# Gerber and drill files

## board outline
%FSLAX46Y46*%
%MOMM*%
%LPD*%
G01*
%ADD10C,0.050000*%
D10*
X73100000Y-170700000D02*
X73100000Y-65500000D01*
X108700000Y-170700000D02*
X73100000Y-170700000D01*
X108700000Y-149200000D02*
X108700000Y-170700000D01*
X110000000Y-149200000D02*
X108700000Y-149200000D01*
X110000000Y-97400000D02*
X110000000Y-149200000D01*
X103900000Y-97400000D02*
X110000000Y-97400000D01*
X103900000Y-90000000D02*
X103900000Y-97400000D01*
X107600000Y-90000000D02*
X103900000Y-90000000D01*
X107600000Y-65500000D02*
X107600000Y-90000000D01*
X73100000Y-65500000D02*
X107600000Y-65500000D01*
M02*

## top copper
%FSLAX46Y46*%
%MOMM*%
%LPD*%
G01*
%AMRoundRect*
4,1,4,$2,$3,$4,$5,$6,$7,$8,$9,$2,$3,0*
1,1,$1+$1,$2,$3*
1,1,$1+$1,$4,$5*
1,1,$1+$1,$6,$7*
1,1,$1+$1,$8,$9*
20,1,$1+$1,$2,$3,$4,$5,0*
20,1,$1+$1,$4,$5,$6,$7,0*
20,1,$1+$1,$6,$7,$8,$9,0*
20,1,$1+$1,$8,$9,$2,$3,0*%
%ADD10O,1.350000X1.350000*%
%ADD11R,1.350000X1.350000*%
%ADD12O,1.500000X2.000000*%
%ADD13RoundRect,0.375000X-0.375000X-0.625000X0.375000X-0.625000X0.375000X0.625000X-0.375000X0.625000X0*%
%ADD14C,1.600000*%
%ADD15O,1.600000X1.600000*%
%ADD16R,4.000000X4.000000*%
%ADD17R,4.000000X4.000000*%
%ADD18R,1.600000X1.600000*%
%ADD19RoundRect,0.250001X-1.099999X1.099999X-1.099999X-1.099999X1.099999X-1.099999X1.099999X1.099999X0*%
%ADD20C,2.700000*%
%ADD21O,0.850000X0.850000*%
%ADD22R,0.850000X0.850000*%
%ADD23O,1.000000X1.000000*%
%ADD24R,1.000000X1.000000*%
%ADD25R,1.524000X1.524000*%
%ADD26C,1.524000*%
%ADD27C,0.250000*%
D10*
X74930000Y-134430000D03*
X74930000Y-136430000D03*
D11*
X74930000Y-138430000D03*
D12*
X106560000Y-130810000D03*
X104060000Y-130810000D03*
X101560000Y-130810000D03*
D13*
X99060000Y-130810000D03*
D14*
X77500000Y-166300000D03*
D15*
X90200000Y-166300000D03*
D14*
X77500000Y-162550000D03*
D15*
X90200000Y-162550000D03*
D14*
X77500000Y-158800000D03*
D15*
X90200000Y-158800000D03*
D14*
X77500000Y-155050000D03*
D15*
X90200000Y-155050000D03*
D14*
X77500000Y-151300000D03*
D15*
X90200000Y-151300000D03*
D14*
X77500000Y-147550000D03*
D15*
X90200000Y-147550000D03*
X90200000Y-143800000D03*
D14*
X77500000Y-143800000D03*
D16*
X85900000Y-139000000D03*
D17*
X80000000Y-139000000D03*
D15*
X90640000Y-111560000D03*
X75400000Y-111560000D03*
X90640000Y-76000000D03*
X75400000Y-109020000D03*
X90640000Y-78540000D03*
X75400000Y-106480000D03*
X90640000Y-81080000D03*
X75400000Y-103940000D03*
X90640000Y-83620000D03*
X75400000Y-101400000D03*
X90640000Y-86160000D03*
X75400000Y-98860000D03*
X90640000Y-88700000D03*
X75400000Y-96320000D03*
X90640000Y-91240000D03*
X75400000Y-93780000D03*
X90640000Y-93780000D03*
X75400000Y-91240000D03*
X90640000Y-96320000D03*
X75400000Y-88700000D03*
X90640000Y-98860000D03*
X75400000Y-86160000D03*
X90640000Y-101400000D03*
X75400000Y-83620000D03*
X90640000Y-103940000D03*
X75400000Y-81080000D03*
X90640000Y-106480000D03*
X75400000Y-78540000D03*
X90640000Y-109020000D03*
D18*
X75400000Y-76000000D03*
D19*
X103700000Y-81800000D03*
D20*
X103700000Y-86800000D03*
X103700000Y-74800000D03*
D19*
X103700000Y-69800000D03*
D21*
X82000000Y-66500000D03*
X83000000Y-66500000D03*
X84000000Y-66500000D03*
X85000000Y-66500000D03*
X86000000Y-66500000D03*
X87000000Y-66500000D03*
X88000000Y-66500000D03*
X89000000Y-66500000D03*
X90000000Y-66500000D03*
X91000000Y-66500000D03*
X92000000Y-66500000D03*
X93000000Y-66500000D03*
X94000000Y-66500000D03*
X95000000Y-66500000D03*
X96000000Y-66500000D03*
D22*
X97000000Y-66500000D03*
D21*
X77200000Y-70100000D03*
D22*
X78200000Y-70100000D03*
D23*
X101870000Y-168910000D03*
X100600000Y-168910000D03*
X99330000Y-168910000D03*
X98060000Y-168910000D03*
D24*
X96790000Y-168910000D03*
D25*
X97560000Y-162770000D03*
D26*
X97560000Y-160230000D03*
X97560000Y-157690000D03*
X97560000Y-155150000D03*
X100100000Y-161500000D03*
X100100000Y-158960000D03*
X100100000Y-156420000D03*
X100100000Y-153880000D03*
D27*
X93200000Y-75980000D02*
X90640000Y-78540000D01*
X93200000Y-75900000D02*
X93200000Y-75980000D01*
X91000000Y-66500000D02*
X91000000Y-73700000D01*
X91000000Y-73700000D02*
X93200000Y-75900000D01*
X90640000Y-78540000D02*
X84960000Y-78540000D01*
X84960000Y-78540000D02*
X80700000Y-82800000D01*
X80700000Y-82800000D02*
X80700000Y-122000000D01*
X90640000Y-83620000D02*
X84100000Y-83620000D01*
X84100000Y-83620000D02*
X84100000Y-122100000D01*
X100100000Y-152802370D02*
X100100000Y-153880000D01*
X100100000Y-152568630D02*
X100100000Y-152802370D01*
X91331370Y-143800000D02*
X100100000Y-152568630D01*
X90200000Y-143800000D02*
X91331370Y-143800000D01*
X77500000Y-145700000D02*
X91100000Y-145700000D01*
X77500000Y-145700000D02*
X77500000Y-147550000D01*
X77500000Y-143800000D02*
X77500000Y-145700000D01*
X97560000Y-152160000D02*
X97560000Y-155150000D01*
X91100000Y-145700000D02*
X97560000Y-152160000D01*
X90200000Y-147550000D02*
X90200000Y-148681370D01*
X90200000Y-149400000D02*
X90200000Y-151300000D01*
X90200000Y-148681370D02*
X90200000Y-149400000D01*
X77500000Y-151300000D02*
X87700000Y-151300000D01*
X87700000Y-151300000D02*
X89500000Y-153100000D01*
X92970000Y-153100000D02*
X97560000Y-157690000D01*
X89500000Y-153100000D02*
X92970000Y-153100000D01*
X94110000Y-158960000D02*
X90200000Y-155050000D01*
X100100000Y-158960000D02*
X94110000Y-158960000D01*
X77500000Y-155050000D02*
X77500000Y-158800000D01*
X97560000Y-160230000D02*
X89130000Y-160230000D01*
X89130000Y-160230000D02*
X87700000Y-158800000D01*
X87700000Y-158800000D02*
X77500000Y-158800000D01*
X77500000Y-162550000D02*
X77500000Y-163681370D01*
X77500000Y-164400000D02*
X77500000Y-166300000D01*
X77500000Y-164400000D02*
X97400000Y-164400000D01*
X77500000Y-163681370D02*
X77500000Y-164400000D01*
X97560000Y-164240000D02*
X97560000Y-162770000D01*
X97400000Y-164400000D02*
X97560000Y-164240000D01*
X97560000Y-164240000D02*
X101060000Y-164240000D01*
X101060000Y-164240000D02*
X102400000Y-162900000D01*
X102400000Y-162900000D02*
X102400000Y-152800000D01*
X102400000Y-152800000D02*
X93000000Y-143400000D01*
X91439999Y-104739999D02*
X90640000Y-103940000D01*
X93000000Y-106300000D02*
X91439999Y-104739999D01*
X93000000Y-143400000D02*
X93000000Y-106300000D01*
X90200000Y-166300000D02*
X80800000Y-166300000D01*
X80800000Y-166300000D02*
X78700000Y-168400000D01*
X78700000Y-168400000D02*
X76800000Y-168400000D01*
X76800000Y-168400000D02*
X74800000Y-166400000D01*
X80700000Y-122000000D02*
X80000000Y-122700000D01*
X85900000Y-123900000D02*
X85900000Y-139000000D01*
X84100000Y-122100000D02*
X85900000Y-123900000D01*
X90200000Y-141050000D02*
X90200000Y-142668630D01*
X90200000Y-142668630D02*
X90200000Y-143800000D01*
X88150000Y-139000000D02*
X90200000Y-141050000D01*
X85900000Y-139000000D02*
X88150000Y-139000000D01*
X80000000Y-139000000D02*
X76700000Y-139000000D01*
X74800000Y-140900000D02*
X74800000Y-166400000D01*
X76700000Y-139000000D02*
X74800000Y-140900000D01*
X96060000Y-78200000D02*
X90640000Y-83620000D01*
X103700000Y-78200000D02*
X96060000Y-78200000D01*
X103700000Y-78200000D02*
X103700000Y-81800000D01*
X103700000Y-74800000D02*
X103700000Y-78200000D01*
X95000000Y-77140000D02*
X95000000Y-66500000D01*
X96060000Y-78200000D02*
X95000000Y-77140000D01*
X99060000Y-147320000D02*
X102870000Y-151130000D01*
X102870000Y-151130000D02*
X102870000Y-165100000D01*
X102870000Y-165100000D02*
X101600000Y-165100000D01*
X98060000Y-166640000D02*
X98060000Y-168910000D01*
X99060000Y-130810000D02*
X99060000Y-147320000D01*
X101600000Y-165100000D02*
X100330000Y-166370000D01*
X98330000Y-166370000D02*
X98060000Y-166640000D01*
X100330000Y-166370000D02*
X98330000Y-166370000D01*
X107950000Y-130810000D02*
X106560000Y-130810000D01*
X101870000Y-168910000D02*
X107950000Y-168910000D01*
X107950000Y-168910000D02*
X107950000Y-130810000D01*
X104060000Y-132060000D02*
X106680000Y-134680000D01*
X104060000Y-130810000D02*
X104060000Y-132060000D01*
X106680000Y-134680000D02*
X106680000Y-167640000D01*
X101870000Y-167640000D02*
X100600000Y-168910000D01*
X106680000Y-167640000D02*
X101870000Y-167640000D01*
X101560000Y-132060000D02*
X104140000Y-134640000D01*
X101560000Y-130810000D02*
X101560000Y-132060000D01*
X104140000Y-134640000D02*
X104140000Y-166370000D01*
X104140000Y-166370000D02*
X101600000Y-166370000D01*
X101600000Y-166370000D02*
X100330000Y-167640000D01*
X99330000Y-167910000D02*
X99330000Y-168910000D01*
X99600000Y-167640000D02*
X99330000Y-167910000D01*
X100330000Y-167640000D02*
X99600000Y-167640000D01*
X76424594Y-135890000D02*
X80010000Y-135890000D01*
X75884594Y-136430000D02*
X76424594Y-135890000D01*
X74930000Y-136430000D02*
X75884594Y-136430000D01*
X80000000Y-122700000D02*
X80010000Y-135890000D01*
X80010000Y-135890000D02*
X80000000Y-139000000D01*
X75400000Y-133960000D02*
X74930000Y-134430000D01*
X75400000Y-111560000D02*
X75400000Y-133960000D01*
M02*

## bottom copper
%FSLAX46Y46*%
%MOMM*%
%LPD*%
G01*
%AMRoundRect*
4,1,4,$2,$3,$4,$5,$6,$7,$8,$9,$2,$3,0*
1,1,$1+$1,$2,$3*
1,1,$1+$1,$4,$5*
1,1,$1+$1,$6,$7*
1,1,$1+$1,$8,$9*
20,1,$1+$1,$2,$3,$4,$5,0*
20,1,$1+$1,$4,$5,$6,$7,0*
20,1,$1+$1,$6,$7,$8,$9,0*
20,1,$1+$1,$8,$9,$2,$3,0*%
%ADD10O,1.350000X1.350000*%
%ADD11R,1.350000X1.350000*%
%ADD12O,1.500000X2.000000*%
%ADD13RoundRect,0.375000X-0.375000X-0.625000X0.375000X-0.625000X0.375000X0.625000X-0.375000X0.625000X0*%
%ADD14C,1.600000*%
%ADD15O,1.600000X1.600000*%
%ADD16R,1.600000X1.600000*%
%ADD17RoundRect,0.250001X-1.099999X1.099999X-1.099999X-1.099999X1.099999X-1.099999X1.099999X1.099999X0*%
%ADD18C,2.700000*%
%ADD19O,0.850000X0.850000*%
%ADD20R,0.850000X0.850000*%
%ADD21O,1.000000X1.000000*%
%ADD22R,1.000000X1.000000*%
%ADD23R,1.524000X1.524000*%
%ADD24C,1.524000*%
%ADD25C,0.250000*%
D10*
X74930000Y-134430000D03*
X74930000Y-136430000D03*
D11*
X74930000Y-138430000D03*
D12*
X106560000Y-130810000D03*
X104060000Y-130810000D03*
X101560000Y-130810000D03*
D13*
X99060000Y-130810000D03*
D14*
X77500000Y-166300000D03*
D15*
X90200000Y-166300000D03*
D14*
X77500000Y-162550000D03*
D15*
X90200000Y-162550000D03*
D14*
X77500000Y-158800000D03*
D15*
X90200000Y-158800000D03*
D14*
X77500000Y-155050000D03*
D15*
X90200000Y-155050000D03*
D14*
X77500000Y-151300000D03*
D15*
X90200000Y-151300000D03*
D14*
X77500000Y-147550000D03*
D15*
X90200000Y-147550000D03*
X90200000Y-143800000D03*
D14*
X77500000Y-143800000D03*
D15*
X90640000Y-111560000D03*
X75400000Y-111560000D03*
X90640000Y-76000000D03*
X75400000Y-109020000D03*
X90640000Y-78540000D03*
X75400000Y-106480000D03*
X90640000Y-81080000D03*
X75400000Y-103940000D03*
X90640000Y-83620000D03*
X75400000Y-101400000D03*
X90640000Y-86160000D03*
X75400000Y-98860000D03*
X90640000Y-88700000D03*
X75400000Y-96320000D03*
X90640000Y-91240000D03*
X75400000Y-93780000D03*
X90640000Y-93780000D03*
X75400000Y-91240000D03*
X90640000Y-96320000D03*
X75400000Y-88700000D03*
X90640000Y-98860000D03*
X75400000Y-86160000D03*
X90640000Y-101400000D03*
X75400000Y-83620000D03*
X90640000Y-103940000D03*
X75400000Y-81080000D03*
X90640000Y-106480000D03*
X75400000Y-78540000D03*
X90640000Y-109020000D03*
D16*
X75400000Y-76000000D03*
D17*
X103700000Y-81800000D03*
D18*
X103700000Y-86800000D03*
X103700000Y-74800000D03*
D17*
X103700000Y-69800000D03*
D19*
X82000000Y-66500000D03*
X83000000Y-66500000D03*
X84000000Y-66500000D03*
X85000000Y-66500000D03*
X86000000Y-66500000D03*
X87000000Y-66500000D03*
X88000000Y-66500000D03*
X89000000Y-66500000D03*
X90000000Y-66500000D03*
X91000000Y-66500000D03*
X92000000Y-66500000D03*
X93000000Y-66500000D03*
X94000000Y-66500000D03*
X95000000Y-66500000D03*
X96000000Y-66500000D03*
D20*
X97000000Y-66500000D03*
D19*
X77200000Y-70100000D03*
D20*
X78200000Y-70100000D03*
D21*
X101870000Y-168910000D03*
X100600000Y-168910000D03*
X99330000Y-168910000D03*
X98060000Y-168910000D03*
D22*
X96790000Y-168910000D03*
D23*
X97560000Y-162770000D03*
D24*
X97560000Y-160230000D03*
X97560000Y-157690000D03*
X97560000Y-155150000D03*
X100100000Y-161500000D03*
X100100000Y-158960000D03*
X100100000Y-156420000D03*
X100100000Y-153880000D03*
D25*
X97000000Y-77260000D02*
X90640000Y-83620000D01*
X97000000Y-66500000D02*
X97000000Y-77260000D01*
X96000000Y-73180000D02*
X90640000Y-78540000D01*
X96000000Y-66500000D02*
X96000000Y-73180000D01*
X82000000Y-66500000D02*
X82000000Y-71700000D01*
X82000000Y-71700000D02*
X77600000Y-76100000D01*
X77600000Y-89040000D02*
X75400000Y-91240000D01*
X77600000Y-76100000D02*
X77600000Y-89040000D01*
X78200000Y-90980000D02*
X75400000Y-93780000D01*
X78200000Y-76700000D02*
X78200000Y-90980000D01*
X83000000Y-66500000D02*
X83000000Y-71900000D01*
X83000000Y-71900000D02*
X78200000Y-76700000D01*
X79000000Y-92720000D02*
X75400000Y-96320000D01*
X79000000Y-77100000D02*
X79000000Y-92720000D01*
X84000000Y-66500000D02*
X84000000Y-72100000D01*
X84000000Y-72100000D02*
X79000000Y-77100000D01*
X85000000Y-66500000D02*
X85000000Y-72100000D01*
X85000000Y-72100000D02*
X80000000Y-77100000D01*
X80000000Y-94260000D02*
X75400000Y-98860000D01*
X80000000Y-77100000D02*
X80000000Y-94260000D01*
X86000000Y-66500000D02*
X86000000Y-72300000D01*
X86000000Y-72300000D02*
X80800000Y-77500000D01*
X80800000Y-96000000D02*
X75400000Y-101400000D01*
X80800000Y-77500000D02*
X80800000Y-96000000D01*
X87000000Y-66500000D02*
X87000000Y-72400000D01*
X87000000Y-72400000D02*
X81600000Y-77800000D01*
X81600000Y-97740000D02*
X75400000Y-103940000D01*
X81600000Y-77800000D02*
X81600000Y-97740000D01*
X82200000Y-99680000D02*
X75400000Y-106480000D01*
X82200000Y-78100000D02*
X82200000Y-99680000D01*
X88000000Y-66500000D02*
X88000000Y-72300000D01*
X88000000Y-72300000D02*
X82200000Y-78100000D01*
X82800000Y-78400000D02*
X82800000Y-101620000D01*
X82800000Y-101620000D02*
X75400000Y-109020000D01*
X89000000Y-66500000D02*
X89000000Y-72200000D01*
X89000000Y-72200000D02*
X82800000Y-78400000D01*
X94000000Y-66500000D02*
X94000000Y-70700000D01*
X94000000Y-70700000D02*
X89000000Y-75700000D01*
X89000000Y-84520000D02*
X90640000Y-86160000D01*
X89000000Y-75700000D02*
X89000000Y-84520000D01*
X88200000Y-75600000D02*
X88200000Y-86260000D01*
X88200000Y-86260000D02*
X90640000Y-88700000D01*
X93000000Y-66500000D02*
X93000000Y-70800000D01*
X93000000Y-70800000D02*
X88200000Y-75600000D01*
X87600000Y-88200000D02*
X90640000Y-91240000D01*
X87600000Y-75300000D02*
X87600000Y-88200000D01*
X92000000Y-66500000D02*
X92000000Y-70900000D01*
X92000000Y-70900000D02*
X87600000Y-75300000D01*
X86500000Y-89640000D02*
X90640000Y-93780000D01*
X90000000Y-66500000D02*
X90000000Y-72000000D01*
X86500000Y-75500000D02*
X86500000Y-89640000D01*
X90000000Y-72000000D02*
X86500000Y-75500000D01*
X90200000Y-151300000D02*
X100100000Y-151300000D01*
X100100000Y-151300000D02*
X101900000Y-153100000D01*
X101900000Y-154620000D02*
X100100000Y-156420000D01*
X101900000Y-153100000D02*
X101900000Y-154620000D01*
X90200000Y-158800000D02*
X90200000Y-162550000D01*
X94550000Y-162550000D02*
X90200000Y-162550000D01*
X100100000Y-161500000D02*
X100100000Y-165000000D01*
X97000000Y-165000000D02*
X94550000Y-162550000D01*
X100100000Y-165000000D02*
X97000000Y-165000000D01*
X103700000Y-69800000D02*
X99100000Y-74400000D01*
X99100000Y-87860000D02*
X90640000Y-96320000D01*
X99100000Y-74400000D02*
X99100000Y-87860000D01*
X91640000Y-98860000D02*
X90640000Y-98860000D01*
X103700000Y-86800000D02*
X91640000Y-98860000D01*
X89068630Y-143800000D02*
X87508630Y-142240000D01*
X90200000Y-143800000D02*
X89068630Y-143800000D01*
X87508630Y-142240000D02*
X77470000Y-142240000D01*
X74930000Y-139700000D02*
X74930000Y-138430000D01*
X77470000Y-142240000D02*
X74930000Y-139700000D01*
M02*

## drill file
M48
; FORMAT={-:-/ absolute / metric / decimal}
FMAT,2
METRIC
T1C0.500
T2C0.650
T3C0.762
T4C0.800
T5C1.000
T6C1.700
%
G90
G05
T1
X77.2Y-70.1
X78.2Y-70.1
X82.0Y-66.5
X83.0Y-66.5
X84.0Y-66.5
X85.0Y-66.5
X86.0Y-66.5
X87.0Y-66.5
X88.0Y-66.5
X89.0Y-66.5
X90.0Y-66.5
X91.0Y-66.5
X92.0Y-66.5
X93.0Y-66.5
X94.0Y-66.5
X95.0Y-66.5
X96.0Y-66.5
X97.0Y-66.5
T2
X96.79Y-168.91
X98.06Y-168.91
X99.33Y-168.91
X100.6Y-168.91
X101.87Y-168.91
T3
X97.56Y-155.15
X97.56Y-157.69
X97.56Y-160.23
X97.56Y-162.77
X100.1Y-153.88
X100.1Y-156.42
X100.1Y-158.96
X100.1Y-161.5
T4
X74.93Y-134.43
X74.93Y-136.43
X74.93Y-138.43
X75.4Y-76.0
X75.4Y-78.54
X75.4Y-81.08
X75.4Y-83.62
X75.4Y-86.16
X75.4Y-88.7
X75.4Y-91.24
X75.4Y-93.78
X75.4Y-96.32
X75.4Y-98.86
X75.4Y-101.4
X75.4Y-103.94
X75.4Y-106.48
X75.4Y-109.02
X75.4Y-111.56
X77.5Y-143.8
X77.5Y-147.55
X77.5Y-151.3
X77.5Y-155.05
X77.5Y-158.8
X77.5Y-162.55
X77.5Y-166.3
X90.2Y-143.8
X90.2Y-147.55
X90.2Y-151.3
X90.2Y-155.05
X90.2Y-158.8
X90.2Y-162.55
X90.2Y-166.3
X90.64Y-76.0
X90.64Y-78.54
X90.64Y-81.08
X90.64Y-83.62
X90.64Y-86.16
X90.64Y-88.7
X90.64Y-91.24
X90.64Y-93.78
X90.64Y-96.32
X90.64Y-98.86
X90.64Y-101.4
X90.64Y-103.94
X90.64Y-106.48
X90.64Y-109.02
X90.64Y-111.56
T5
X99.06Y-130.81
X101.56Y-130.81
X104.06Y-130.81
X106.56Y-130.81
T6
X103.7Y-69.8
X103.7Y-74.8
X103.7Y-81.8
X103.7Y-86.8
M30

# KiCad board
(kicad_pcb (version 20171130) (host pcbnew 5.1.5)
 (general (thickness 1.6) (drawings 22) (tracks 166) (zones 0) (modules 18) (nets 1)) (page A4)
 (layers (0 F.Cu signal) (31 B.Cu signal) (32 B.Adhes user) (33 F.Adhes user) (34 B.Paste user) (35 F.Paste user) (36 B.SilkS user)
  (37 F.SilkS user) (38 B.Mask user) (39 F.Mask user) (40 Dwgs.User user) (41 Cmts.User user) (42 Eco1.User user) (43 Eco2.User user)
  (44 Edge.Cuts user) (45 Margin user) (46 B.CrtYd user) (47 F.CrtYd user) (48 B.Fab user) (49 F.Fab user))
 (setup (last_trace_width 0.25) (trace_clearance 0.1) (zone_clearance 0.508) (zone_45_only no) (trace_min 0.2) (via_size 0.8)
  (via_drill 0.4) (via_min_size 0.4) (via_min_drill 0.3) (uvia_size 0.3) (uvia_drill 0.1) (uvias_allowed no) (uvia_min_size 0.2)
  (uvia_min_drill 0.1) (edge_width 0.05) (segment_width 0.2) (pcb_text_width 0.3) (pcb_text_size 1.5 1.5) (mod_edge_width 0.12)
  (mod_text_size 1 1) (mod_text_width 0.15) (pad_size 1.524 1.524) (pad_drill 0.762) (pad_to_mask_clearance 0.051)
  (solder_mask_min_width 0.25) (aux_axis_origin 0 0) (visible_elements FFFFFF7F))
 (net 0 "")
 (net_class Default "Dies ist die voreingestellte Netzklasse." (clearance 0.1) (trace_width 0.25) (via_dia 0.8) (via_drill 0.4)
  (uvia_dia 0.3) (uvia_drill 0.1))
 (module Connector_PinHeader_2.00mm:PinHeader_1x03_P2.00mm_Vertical (layer F.Cu) (at 74.93 138.43 180)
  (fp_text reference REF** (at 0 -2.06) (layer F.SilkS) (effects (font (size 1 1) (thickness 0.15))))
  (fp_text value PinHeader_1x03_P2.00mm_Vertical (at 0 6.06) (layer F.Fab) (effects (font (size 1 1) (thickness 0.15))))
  (pad 3 thru_hole oval (at 0 4 180) (size 1.35 1.35) (drill 0.8) (layers *.Cu *.Mask))
  (pad 2 thru_hole oval (at 0 2 180) (size 1.35 1.35) (drill 0.8) (layers *.Cu *.Mask))
  (pad 1 thru_hole rect (at 0 0 180) (size 1.35 1.35) (drill 0.8) (layers *.Cu *.Mask)))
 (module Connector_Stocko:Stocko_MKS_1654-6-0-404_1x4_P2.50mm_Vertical (layer F.Cu) (at 99.06 130.81)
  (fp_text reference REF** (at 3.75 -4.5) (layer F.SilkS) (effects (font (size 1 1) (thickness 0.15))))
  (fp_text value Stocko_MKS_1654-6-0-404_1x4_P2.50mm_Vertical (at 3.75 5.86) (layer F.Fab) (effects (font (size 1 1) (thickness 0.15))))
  (pad 4 thru_hole oval (at 7.5 0) (size 1.5 2) (drill 1) (layers *.Cu *.Mask))
  (pad 3 thru_hole oval (at 5 0) (size 1.5 2) (drill 1) (layers *.Cu *.Mask))
  (pad 2 thru_hole oval (at 2.5 0) (size 1.5 2) (drill 1) (layers *.Cu *.Mask))
  (pad 1 thru_hole roundrect (at 0 0) (size 1.5 2) (drill 1) (layers *.Cu *.Mask) (roundrect_rratio 0.25)))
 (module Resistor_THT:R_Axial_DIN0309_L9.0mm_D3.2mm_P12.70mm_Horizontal (layer F.Cu) (at 77.5 166.3)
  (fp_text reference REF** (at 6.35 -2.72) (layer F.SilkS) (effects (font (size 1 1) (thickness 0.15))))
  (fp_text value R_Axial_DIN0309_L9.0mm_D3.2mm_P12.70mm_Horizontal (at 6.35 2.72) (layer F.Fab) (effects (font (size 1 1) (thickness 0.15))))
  (pad 1 thru_hole circle (at 0 0) (size 1.6 1.6) (drill 0.8) (layers *.Cu *.Mask))
  (pad 2 thru_hole oval (at 12.7 0) (size 1.6 1.6) (drill 0.8) (layers *.Cu *.Mask)))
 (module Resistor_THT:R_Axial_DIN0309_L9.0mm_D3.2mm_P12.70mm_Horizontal (layer F.Cu) (at 77.5 162.55)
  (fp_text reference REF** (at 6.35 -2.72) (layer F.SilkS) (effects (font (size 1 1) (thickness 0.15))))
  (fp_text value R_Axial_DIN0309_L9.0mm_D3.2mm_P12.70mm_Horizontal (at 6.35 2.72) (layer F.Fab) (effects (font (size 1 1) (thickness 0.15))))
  (pad 1 thru_hole circle (at 0 0) (size 1.6 1.6) (drill 0.8) (layers *.Cu *.Mask))
  (pad 2 thru_hole oval (at 12.7 0) (size 1.6 1.6) (drill 0.8) (layers *.Cu *.Mask)))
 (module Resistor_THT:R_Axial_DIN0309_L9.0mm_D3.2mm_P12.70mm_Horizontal (layer F.Cu) (at 77.5 158.8)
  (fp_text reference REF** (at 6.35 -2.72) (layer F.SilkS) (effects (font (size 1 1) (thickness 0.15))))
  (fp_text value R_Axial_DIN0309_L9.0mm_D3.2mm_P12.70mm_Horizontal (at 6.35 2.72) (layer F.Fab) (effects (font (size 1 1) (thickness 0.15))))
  (pad 1 thru_hole circle (at 0 0) (size 1.6 1.6) (drill 0.8) (layers *.Cu *.Mask))
  (pad 2 thru_hole oval (at 12.7 0) (size 1.6 1.6) (drill 0.8) (layers *.Cu *.Mask)))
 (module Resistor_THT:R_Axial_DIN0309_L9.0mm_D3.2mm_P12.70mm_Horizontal (layer F.Cu) (at 77.5 155.05)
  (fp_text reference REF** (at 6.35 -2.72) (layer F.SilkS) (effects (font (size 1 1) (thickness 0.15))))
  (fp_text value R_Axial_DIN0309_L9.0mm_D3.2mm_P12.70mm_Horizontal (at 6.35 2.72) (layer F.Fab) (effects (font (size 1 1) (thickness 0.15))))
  (pad 1 thru_hole circle (at 0 0) (size 1.6 1.6) (drill 0.8) (layers *.Cu *.Mask))
  (pad 2 thru_hole oval (at 12.7 0) (size 1.6 1.6) (drill 0.8) (layers *.Cu *.Mask)))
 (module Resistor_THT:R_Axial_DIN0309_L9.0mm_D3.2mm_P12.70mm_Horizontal (layer F.Cu) (at 77.5 151.3)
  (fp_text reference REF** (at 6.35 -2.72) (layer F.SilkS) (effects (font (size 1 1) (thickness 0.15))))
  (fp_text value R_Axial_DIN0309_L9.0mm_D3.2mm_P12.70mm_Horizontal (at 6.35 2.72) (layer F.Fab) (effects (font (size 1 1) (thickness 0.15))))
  (pad 1 thru_hole circle (at 0 0) (size 1.6 1.6) (drill 0.8) (layers *.Cu *.Mask))
  (pad 2 thru_hole oval (at 12.7 0) (size 1.6 1.6) (drill 0.8) (layers *.Cu *.Mask)))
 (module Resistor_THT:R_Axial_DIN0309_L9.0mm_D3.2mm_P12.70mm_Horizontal (layer F.Cu) (at 77.5 147.55)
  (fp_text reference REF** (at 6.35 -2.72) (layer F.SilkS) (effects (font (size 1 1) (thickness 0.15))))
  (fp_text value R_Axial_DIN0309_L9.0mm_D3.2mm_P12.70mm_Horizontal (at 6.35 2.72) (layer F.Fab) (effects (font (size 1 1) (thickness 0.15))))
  (pad 1 thru_hole circle (at 0 0) (size 1.6 1.6) (drill 0.8) (layers *.Cu *.Mask))
  (pad 2 thru_hole oval (at 12.7 0) (size 1.6 1.6) (drill 0.8) (layers *.Cu *.Mask)))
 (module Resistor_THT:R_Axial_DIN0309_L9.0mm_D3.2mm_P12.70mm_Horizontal (layer F.Cu) (at 77.5 143.8)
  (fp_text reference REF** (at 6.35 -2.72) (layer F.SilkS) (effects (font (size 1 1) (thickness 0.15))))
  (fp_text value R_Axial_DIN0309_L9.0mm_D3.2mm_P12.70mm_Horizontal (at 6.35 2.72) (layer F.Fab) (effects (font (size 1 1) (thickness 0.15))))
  (pad 2 thru_hole oval (at 12.7 0) (size 1.6 1.6) (drill 0.8) (layers *.Cu *.Mask))
  (pad 1 thru_hole circle (at 0 0) (size 1.6 1.6) (drill 0.8) (layers *.Cu *.Mask)))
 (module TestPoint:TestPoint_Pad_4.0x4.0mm (layer F.Cu) (at 85.9 139)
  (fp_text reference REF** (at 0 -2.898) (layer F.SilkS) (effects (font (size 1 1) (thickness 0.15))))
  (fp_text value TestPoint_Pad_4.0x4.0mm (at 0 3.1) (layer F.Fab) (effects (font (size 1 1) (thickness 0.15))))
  (pad + connect rect (at 0 0) (size 4 4) (layers F.Cu F.Mask)))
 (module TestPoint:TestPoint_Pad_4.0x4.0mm (layer F.Cu) (at 80 139)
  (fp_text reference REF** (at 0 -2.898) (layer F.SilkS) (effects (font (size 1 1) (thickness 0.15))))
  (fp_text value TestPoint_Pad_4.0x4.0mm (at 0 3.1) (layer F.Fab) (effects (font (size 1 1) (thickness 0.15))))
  (pad - smd rect (at 0 0) (size 4 4) (layers F.Cu F.Mask)))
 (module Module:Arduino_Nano (layer F.Cu) (at 75.4 76)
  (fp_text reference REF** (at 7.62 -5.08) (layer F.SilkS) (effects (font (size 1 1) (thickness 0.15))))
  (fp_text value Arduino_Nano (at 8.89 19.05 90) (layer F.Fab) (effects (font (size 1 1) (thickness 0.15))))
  (pad 16 thru_hole oval (at 15.24 35.56) (size 1.6 1.6) (drill 0.8) (layers *.Cu *.Mask))
  (pad 15 thru_hole oval (at 0 35.56) (size 1.6 1.6) (drill 0.8) (layers *.Cu *.Mask))
  (pad 30 thru_hole oval (at 15.24 0) (size 1.6 1.6) (drill 0.8) (layers *.Cu *.Mask))
  (pad 14 thru_hole oval (at 0 33.02) (size 1.6 1.6) (drill 0.8) (layers *.Cu *.Mask))
  (pad 29 thru_hole oval (at 15.24 2.54) (size 1.6 1.6) (drill 0.8) (layers *.Cu *.Mask))
  (pad 13 thru_hole oval (at 0 30.48) (size 1.6 1.6) (drill 0.8) (layers *.Cu *.Mask))
  (pad 28 thru_hole oval (at 15.24 5.08) (size 1.6 1.6) (drill 0.8) (layers *.Cu *.Mask))
  (pad 12 thru_hole oval (at 0 27.94) (size 1.6 1.6) (drill 0.8) (layers *.Cu *.Mask))
  (pad 27 thru_hole oval (at 15.24 7.62) (size 1.6 1.6) (drill 0.8) (layers *.Cu *.Mask))
  (pad 11 thru_hole oval (at 0 25.4) (size 1.6 1.6) (drill 0.8) (layers *.Cu *.Mask))
  (pad 26 thru_hole oval (at 15.24 10.16) (size 1.6 1.6) (drill 0.8) (layers *.Cu *.Mask))
  (pad 10 thru_hole oval (at 0 22.86) (size 1.6 1.6) (drill 0.8) (layers *.Cu *.Mask))
  (pad 25 thru_hole oval (at 15.24 12.7) (size 1.6 1.6) (drill 0.8) (layers *.Cu *.Mask))
  (pad 9 thru_hole oval (at 0 20.32) (size 1.6 1.6) (drill 0.8) (layers *.Cu *.Mask))
  (pad 24 thru_hole oval (at 15.24 15.24) (size 1.6 1.6) (drill 0.8) (layers *.Cu *.Mask))
  (pad 8 thru_hole oval (at 0 17.78) (size 1.6 1.6) (drill 0.8) (layers *.Cu *.Mask))
  (pad 23 thru_hole oval (at 15.24 17.78) (size 1.6 1.6) (drill 0.8) (layers *.Cu *.Mask))
  (pad 7 thru_hole oval (at 0 15.24) (size 1.6 1.6) (drill 0.8) (layers *.Cu *.Mask))
  (pad 22 thru_hole oval (at 15.24 20.32) (size 1.6 1.6) (drill 0.8) (layers *.Cu *.Mask))
  (pad 6 thru_hole oval (at 0 12.7) (size 1.6 1.6) (drill 0.8) (layers *.Cu *.Mask))
  (pad 21 thru_hole oval (at 15.24 22.86) (size 1.6 1.6) (drill 0.8) (layers *.Cu *.Mask))
  (pad 5 thru_hole oval (at 0 10.16) (size 1.6 1.6) (drill 0.8) (layers *.Cu *.Mask))
  (pad 20 thru_hole oval (at 15.24 25.4) (size 1.6 1.6) (drill 0.8) (layers *.Cu *.Mask))
  (pad 4 thru_hole oval (at 0 7.62) (size 1.6 1.6) (drill 0.8) (layers *.Cu *.Mask))
  (pad 19 thru_hole oval (at 15.24 27.94) (size 1.6 1.6) (drill 0.8) (layers *.Cu *.Mask))
  (pad 3 thru_hole oval (at 0 5.08) (size 1.6 1.6) (drill 0.8) (layers *.Cu *.Mask))
  (pad 18 thru_hole oval (at 15.24 30.48) (size 1.6 1.6) (drill 0.8) (layers *.Cu *.Mask))
  (pad 2 thru_hole oval (at 0 2.54) (size 1.6 1.6) (drill 0.8) (layers *.Cu *.Mask))
  (pad 17 thru_hole oval (at 15.24 33.02) (size 1.6 1.6) (drill 0.8) (layers *.Cu *.Mask))
  (pad 1 thru_hole rect (at 0 0) (size 1.6 1.6) (drill 0.8) (layers *.Cu *.Mask)))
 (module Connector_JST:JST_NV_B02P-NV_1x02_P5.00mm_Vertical (layer F.Cu) (at 103.7 81.8 270)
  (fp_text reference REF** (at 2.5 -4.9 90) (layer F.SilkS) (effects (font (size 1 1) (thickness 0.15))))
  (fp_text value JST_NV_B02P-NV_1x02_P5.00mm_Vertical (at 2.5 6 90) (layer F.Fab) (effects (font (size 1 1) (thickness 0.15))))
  (pad 1 thru_hole roundrect (at 0 0 270) (size 2.7 2.7) (drill 1.7) (layers *.Cu *.Mask) (roundrect_rratio 0.09259299999999999))
  (pad 2 thru_hole circle (at 5 0 270) (size 2.7 2.7) (drill 1.7) (layers *.Cu *.Mask)))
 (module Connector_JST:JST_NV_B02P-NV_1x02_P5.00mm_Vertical (layer F.Cu) (at 103.7 69.8 270)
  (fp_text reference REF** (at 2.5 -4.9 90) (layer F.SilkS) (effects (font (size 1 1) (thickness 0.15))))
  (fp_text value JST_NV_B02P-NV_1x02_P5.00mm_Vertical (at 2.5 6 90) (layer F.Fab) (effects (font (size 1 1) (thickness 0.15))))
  (pad 2 thru_hole circle (at 5 0 270) (size 2.7 2.7) (drill 1.7) (layers *.Cu *.Mask))
  (pad 1 thru_hole roundrect (at 0 0 270) (size 2.7 2.7) (drill 1.7) (layers *.Cu *.Mask) (roundrect_rratio 0.09259299999999999)))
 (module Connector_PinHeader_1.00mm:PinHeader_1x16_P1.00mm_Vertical (layer F.Cu) (at 97 66.5 270)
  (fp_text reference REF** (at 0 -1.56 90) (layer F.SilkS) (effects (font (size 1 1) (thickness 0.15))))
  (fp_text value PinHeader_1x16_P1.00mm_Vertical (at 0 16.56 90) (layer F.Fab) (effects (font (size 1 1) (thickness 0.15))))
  (pad 16 thru_hole oval (at 0 15 270) (size 0.85 0.85) (drill 0.5) (layers *.Cu *.Mask))
  (pad 15 thru_hole oval (at 0 14 270) (size 0.85 0.85) (drill 0.5) (layers *.Cu *.Mask))
  (pad 14 thru_hole oval (at 0 13 270) (size 0.85 0.85) (drill 0.5) (layers *.Cu *.Mask))
  (pad 13 thru_hole oval (at 0 12 270) (size 0.85 0.85) (drill 0.5) (layers *.Cu *.Mask))
  (pad 12 thru_hole oval (at 0 11 270) (size 0.85 0.85) (drill 0.5) (layers *.Cu *.Mask))
  (pad 11 thru_hole oval (at 0 10 270) (size 0.85 0.85) (drill 0.5) (layers *.Cu *.Mask))
  (pad 10 thru_hole oval (at 0 9 270) (size 0.85 0.85) (drill 0.5) (layers *.Cu *.Mask))
  (pad 9 thru_hole oval (at 0 8 270) (size 0.85 0.85) (drill 0.5) (layers *.Cu *.Mask))
  (pad 8 thru_hole oval (at 0 7 270) (size 0.85 0.85) (drill 0.5) (layers *.Cu *.Mask))
  (pad 7 thru_hole oval (at 0 6 270) (size 0.85 0.85) (drill 0.5) (layers *.Cu *.Mask))
  (pad 6 thru_hole oval (at 0 5 270) (size 0.85 0.85) (drill 0.5) (layers *.Cu *.Mask))
  (pad 5 thru_hole oval (at 0 4 270) (size 0.85 0.85) (drill 0.5) (layers *.Cu *.Mask))
  (pad 4 thru_hole oval (at 0 3 270) (size 0.85 0.85) (drill 0.5) (layers *.Cu *.Mask))
  (pad 3 thru_hole oval (at 0 2 270) (size 0.85 0.85) (drill 0.5) (layers *.Cu *.Mask))
  (pad 2 thru_hole oval (at 0 1 270) (size 0.85 0.85) (drill 0.5) (layers *.Cu *.Mask))
  (pad 1 thru_hole rect (at 0 0 270) (size 0.85 0.85) (drill 0.5) (layers *.Cu *.Mask)))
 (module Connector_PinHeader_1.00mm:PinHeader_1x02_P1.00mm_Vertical (layer F.Cu) (at 78.2 70.1 270)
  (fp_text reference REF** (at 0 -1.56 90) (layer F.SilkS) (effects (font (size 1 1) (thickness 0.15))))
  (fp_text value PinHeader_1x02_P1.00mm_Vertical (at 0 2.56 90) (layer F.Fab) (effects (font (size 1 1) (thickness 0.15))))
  (pad 2 thru_hole oval (at 0 1 270) (size 0.85 0.85) (drill 0.5) (layers *.Cu *.Mask))
  (pad 1 thru_hole rect (at 0 0 270) (size 0.85 0.85) (drill 0.5) (layers *.Cu *.Mask)))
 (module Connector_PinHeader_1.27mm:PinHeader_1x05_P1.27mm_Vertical (layer F.Cu) (at 96.79 168.91 90)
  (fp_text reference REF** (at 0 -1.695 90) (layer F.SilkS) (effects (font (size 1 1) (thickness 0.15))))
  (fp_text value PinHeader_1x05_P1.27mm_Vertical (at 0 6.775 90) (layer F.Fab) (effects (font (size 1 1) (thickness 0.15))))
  (pad 5 thru_hole oval (at 0 5.08 90) (size 1 1) (drill 0.65) (layers *.Cu *.Mask))
  (pad 4 thru_hole oval (at 0 3.81 90) (size 1 1) (drill 0.65) (layers *.Cu *.Mask))
  (pad 3 thru_hole oval (at 0 2.54 90) (size 1 1) (drill 0.65) (layers *.Cu *.Mask))
  (pad 2 thru_hole oval (at 0 1.27 90) (size 1 1) (drill 0.65) (layers *.Cu *.Mask))
  (pad 1 thru_hole rect (at 0 0 90) (size 1 1) (drill 0.65) (layers *.Cu *.Mask)))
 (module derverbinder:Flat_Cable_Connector (layer F.Cu) (at 96.29 157.69 90)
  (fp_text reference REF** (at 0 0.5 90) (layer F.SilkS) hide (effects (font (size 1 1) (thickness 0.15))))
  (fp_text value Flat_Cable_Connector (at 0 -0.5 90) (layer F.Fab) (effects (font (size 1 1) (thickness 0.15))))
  (pad 1 thru_hole rect (at -5.08 1.27 90) (size 1.524 1.524) (drill 0.762) (layers *.Cu *.Mask))
  (pad 3 thru_hole circle (at -2.54 1.27 90) (size 1.524 1.524) (drill 0.762) (layers *.Cu *.Mask))
  (pad 5 thru_hole circle (at 0 1.27 90) (size 1.524 1.524) (drill 0.762) (layers *.Cu *.Mask))
  (pad 7 thru_hole circle (at 2.54 1.27 90) (size 1.524 1.524) (drill 0.762) (layers *.Cu *.Mask))
  (pad 2 thru_hole circle (at -3.81 3.81 90) (size 1.524 1.524) (drill 0.762) (layers *.Cu *.Mask))
  (pad 4 thru_hole circle (at -1.27 3.81 90) (size 1.524 1.524) (drill 0.762) (layers *.Cu *.Mask))
  (pad 6 thru_hole circle (at 1.27 3.81 90) (size 1.524 1.524) (drill 0.762) (layers *.Cu *.Mask))
  (pad 8 thru_hole circle (at 3.81 3.81 90) (size 1.524 1.524) (drill 0.762) (layers *.Cu *.Mask)))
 (gr_line (start 73.1 170.7) (end 73.1 65.5) (layer Edge.Cuts) (width 0.05))
 (gr_line (start 108.7 170.7) (end 73.1 170.7) (layer Edge.Cuts) (width 0.05))
 (gr_line (start 108.7 149.2) (end 108.7 170.7) (layer Edge.Cuts) (width 0.05))
 (gr_line (start 110 149.2) (end 108.7 149.2) (layer Edge.Cuts) (width 0.05))
 (gr_line (start 110 97.4) (end 110 149.2) (layer Edge.Cuts) (width 0.05))
 (gr_line (start 103.9 97.4) (end 110 97.4) (layer Edge.Cuts) (width 0.05))
 (gr_line (start 103.9 90) (end 103.9 97.4) (layer Edge.Cuts) (width 0.05))
 (gr_line (start 107.6 90) (end 103.9 90) (layer Edge.Cuts) (width 0.05))
 (gr_line (start 107.6 65.5) (end 107.6 90) (layer Edge.Cuts) (width 0.05))
 (gr_line (start 73.1 65.5) (end 107.6 65.5) (layer Edge.Cuts) (width 0.05))
 (segment (start 97 77.26) (end 90.64 83.62) (width 0.25) (layer B.Cu) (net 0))
 (segment (start 97 66.5) (end 97 77.26) (width 0.25) (layer B.Cu) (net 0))
 (segment (start 96 73.18) (end 90.64 78.54) (width 0.25) (layer B.Cu) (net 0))
 (segment (start 96 66.5) (end 96 73.18) (width 0.25) (layer B.Cu) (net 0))
 (segment (start 82 66.5) (end 82 71.7) (width 0.25) (layer B.Cu) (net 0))
 (segment (start 82 71.7) (end 77.6 76.1) (width 0.25) (layer B.Cu) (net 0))
 (segment (start 77.6 89.04) (end 75.4 91.24) (width 0.25) (layer B.Cu) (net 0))
 (segment (start 77.6 76.1) (end 77.6 89.04) (width 0.25) (layer B.Cu) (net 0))
 (segment (start 78.2 90.98) (end 75.4 93.78) (width 0.25) (layer B.Cu) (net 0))
 (segment (start 78.2 76.7) (end 78.2 90.98) (width 0.25) (layer B.Cu) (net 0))
 (segment (start 83 66.5) (end 83 71.9) (width 0.25) (layer B.Cu) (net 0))
 (segment (start 83 71.9) (end 78.2 76.7) (width 0.25) (layer B.Cu) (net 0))
 (segment (start 79 92.72) (end 75.4 96.32) (width 0.25) (layer B.Cu) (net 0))
 (segment (start 79 77.1) (end 79 92.72) (width 0.25) (layer B.Cu) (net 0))
 (segment (start 84 66.5) (end 84 72.1) (width 0.25) (layer B.Cu) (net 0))
 (segment (start 84 72.1) (end 79 77.1) (width 0.25) (layer B.Cu) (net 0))
 (segment (start 85 66.5) (end 85 72.1) (width 0.25) (layer B.Cu) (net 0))
 (segment (start 85 72.1) (end 80 77.1) (width 0.25) (layer B.Cu) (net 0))
 (segment (start 80 94.26) (end 75.4 98.86) (width 0.25) (layer B.Cu) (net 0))
 (segment (start 80 77.1) (end 80 94.26) (width 0.25) (layer B.Cu) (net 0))
 (segment (start 86 66.5) (end 86 72.3) (width 0.25) (layer B.Cu) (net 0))
 (segment (start 86 72.3) (end 80.8 77.5) (width 0.25) (layer B.Cu) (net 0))
 (segment (start 80.8 96) (end 75.4 101.4) (width 0.25) (layer B.Cu) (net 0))
 (segment (start 80.8 77.5) (end 80.8 96) (width 0.25) (layer B.Cu) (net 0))
 (segment (start 87 66.5) (end 87 72.4) (width 0.25) (layer B.Cu) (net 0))
 (segment (start 87 72.4) (end 81.6 77.8) (width 0.25) (layer B.Cu) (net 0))
 (segment (start 81.6 97.74) (end 75.4 103.94) (width 0.25) (layer B.Cu) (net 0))
 (segment (start 81.6 77.8) (end 81.6 97.74) (width 0.25) (layer B.Cu) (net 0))
 (segment (start 82.2 99.68) (end 75.4 106.48) (width 0.25) (layer B.Cu) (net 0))
 (segment (start 82.2 78.1) (end 82.2 99.68) (width 0.25) (layer B.Cu) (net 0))
 (segment (start 88 66.5) (end 88 72.3) (width 0.25) (layer B.Cu) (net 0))
 (segment (start 88 72.3) (end 82.2 78.1) (width 0.25) (layer B.Cu) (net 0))
 (segment (start 82.8 78.4) (end 82.8 101.62) (width 0.25) (layer B.Cu) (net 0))
 (segment (start 82.8 101.62) (end 75.4 109.02) (width 0.25) (layer B.Cu) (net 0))
 (segment (start 89 66.5) (end 89 72.2) (width 0.25) (layer B.Cu) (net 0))
 (segment (start 89 72.2) (end 82.8 78.4) (width 0.25) (layer B.Cu) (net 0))
 (segment (start 93.2 75.98) (end 90.64 78.54) (width 0.25) (layer F.Cu) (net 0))
 (segment (start 93.2 75.9) (end 93.2 75.98) (width 0.25) (layer F.Cu) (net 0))
 (segment (start 91 66.5) (end 91 73.7) (width 0.25) (layer F.Cu) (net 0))
 (segment (start 91 73.7) (end 93.2 75.9) (width 0.25) (layer F.Cu) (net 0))
 (segment (start 94 66.5) (end 94 70.7) (width 0.25) (layer B.Cu) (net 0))
 (segment (start 94 70.7) (end 89 75.7) (width 0.25) (layer B.Cu) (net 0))
 (segment (start 89 84.52) (end 90.64 86.16) (width 0.25) (layer B.Cu) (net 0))
 (segment (start 89 75.7) (end 89 84.52) (width 0.25) (layer B.Cu) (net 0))
 (segment (start 88.2 75.6) (end 88.2 86.26) (width 0.25) (layer B.Cu) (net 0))
 (segment (start 88.2 86.26) (end 90.64 88.7) (width 0.25) (layer B.Cu) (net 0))
 (segment (start 93 66.5) (end 93 70.8) (width 0.25) (layer B.Cu) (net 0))
 (segment (start 93 70.8) (end 88.2 75.6) (width 0.25) (layer B.Cu) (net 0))
 (segment (start 87.6 88.2) (end 90.64 91.24) (width 0.25) (layer B.Cu) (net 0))
 (segment (start 87.6 75.3) (end 87.6 88.2) (width 0.25) (layer B.Cu) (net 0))
 (segment (start 92 66.5) (end 92 70.9) (width 0.25) (layer B.Cu) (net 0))
 (segment (start 92 70.9) (end 87.6 75.3) (width 0.25) (layer B.Cu) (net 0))
 (segment (start 86.5 89.64) (end 90.64 93.78) (width 0.25) (layer B.Cu) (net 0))
 (segment (start 90 66.5) (end 90 72) (width 0.25) (layer B.Cu) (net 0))
 (segment (start 86.5 75.5) (end 86.5 89.64) (width 0.25) (layer B.Cu) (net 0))
 (segment (start 90 72) (end 86.5 75.5) (width 0.25) (layer B.Cu) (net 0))
 (segment (start 90.64 78.54) (end 84.96 78.54) (width 0.25) (layer F.Cu) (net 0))
 (segment (start 84.96 78.54) (end 80.7 82.8) (width 0.25) (layer F.Cu) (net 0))
 (segment (start 80.7 82.8) (end 80.7 122) (width 0.25) (layer F.Cu) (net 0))
 (segment (start 90.64 83.62) (end 84.1 83.62) (width 0.25) (layer F.Cu) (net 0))
 (segment (start 84.1 83.62) (end 84.1 122.1) (width 0.25) (layer F.Cu) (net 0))
 (segment (start 100.1 152.80237) (end 100.1 153.88) (width 0.25) (layer F.Cu) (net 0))
 (segment (start 100.1 152.56863) (end 100.1 152.80237) (width 0.25) (layer F.Cu) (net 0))
 (segment (start 91.33137 143.8) (end 100.1 152.56863) (width 0.25) (layer F.Cu) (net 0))
 (segment (start 90.2 143.8) (end 91.33137 143.8) (width 0.25) (layer F.Cu) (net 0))
 (segment (start 77.5 145.7) (end 91.1 145.7) (width 0.25) (layer F.Cu) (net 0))
 (segment (start 77.5 145.7) (end 77.5 147.55) (width 0.25) (layer F.Cu) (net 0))
 (segment (start 77.5 143.8) (end 77.5 145.7) (width 0.25) (layer F.Cu) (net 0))
 (segment (start 97.56 152.16) (end 97.56 155.15) (width 0.25) (layer F.Cu) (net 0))
 (segment (start 91.1 145.7) (end 97.56 152.16) (width 0.25) (layer F.Cu) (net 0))
 (segment (start 90.2 147.55) (end 90.2 148.68137) (width 0.25) (layer F.Cu) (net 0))
 (segment (start 90.2 149.4) (end 90.2 151.3) (width 0.25) (layer F.Cu) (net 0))
 (segment (start 90.2 148.68137) (end 90.2 149.4) (width 0.25) (layer F.Cu) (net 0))
 (segment (start 90.2 151.3) (end 100.1 151.3) (width 0.25) (layer B.Cu) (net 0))
 (segment (start 100.1 151.3) (end 101.9 153.1) (width 0.25) (layer B.Cu) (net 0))
 (segment (start 101.9 154.62) (end 100.1 156.42) (width 0.25) (layer B.Cu) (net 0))
 (segment (start 101.9 153.1) (end 101.9 154.62) (width 0.25) (layer B.Cu) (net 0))
 (segment (start 77.5 151.3) (end 87.7 151.3) (width 0.25) (layer F.Cu) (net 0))
 (segment (start 87.7 151.3) (end 89.5 153.1) (width 0.25) (layer F.Cu) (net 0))
 (segment (start 92.97 153.1) (end 97.56 157.69) (width 0.25) (layer F.Cu) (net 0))
 (segment (start 89.5 153.1) (end 92.97 153.1) (width 0.25) (layer F.Cu) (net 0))
 (segment (start 94.11 158.96) (end 90.2 155.05) (width 0.25) (layer F.Cu) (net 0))
 (segment (start 100.1 158.96) (end 94.11 158.96) (width 0.25) (layer F.Cu) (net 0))
 (segment (start 77.5 155.05) (end 77.5 158.8) (width 0.25) (layer F.Cu) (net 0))
 (segment (start 97.56 160.23) (end 89.13 160.23) (width 0.25) (layer F.Cu) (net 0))
 (segment (start 89.13 160.23) (end 87.7 158.8) (width 0.25) (layer F.Cu) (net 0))
 (segment (start 87.7 158.8) (end 77.5 158.8) (width 0.25) (layer F.Cu) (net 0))
 (segment (start 90.2 158.8) (end 90.2 162.55) (width 0.25) (layer B.Cu) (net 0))
 (segment (start 94.55 162.55) (end 90.2 162.55) (width 0.25) (layer B.Cu) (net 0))
 (segment (start 100.1 161.5) (end 100.1 165) (width 0.25) (layer B.Cu) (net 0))
 (segment (start 97 165) (end 94.55 162.55) (width 0.25) (layer B.Cu) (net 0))
 (segment (start 100.1 165) (end 97 165) (width 0.25) (layer B.Cu) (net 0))
 (segment (start 77.5 162.55) (end 77.5 163.68137) (width 0.25) (layer F.Cu) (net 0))
 (segment (start 77.5 164.4) (end 77.5 166.3) (width 0.25) (layer F.Cu) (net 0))
 (segment (start 77.5 164.4) (end 97.4 164.4) (width 0.25) (layer F.Cu) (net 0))
 (segment (start 77.5 163.68137) (end 77.5 164.4) (width 0.25) (layer F.Cu) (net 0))
 (segment (start 97.56 164.24) (end 97.56 162.77) (width 0.25) (layer F.Cu) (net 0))
 (segment (start 97.4 164.4) (end 97.56 164.24) (width 0.25) (layer F.Cu) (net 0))
 (segment (start 97.56 164.24) (end 101.06 164.24) (width 0.25) (layer F.Cu) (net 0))
 (segment (start 101.06 164.24) (end 102.4 162.9) (width 0.25) (layer F.Cu) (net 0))
 (segment (start 102.4 162.9) (end 102.4 152.8) (width 0.25) (layer F.Cu) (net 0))
 (segment (start 102.4 152.8) (end 93 143.4) (width 0.25) (layer F.Cu) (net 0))
 (segment (start 91.439999 104.739999) (end 90.64 103.94) (width 0.25) (layer F.Cu) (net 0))
 (segment (start 93 106.3) (end 91.439999 104.739999) (width 0.25) (layer F.Cu) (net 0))
 (segment (start 93 143.4) (end 93 106.3) (width 0.25) (layer F.Cu) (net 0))
 (segment (start 90.2 166.3) (end 80.8 166.3) (width 0.25) (layer F.Cu) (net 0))
 (segment (start 80.8 166.3) (end 78.7 168.4) (width 0.25) (layer F.Cu) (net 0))
 (segment (start 78.7 168.4) (end 76.8 168.4) (width 0.25) (layer F.Cu) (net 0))
 (segment (start 76.8 168.4) (end 74.8 166.4) (width 0.25) (layer F.Cu) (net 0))
 (segment (start 80.7 122) (end 80 122.7) (width 0.25) (layer F.Cu) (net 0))
 (segment (start 85.9 123.9) (end 85.9 139) (width 0.25) (layer F.Cu) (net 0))
 (segment (start 84.1 122.1) (end 85.9 123.9) (width 0.25) (layer F.Cu) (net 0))
 (segment (start 90.2 141.05) (end 90.2 142.66863) (width 0.25) (layer F.Cu) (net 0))
 (segment (start 90.2 142.66863) (end 90.2 143.8) (width 0.25) (layer F.Cu) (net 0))
 (segment (start 88.15 139) (end 90.2 141.05) (width 0.25) (layer F.Cu) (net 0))
 (segment (start 85.9 139) (end 88.15 139) (width 0.25) (layer F.Cu) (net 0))
 (segment (start 80 139) (end 76.7 139) (width 0.25) (layer F.Cu) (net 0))
 (segment (start 74.8 140.9) (end 74.8 166.4) (width 0.25) (layer F.Cu) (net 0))
 (segment (start 76.7 139) (end 74.8 140.9) (width 0.25) (layer F.Cu) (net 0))
 (segment (start 96.06 78.2) (end 90.64 83.62) (width 0.25) (layer F.Cu) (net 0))
 (segment (start 103.7 78.2) (end 96.06 78.2) (width 0.25) (layer F.Cu) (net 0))
 (segment (start 103.7 78.2) (end 103.7 81.8) (width 0.25) (layer F.Cu) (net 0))
 (segment (start 103.7 74.8) (end 103.7 78.2) (width 0.25) (layer F.Cu) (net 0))
 (segment (start 103.7 69.8) (end 99.1 74.4) (width 0.25) (layer B.Cu) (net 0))
 (segment (start 99.1 87.86) (end 90.64 96.32) (width 0.25) (layer B.Cu) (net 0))
 (segment (start 99.1 74.4) (end 99.1 87.86) (width 0.25) (layer B.Cu) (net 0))
 (segment (start 91.64 98.86) (end 90.64 98.86) (width 0.25) (layer B.Cu) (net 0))
 (segment (start 103.7 86.8) (end 91.64 98.86) (width 0.25) (layer B.Cu) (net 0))
 (segment (start 95 77.14) (end 95 66.5) (width 0.25) (layer F.Cu) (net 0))
 (segment (start 96.06 78.2) (end 95 77.14) (width 0.25) (layer F.Cu) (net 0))
 (segment (start 99.06 147.32) (end 102.87 151.13) (width 0.25) (layer F.Cu) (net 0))
 (segment (start 102.87 151.13) (end 102.87 165.1) (width 0.25) (layer F.Cu) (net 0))
 (segment (start 102.87 165.1) (end 101.6 165.1) (width 0.25) (layer F.Cu) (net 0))
 (segment (start 98.06 166.64) (end 98.06 168.91) (width 0.25) (layer F.Cu) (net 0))
 (segment (start 99.06 130.81) (end 99.06 147.32) (width 0.25) (layer F.Cu) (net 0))
 (segment (start 101.6 165.1) (end 100.33 166.37) (width 0.25) (layer F.Cu) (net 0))
 (segment (start 98.33 166.37) (end 98.06 166.64) (width 0.25) (layer F.Cu) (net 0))
 (segment (start 100.33 166.37) (end 98.33 166.37) (width 0.25) (layer F.Cu) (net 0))
 (segment (start 107.95 130.81) (end 106.56 130.81) (width 0.25) (layer F.Cu) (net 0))
 (segment (start 101.87 168.91) (end 107.95 168.91) (width 0.25) (layer F.Cu) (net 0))
 (segment (start 107.95 168.91) (end 107.95 130.81) (width 0.25) (layer F.Cu) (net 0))
 (segment (start 104.06 132.06) (end 106.68 134.68) (width 0.25) (layer F.Cu) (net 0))
 (segment (start 104.06 130.81) (end 104.06 132.06) (width 0.25) (layer F.Cu) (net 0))
 (segment (start 106.68 134.68) (end 106.68 167.64) (width 0.25) (layer F.Cu) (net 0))
 (segment (start 101.87 167.64) (end 100.6 168.91) (width 0.25) (layer F.Cu) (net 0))
 (segment (start 106.68 167.64) (end 101.87 167.64) (width 0.25) (layer F.Cu) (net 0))
 (segment (start 101.56 132.06) (end 104.14 134.64) (width 0.25) (layer F.Cu) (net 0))
 (segment (start 101.56 130.81) (end 101.56 132.06) (width 0.25) (layer F.Cu) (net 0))
 (segment (start 104.14 134.64) (end 104.14 166.37) (width 0.25) (layer F.Cu) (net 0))
 (segment (start 104.14 166.37) (end 101.6 166.37) (width 0.25) (layer F.Cu) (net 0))
 (segment (start 101.6 166.37) (end 100.33 167.64) (width 0.25) (layer F.Cu) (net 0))
 (segment (start 99.33 167.91) (end 99.33 168.91) (width 0.25) (layer F.Cu) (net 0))
 (segment (start 99.6 167.64) (end 99.33 167.91) (width 0.25) (layer F.Cu) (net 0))
 (segment (start 100.33 167.64) (end 99.6 167.64) (width 0.25) (layer F.Cu) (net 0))
 (segment (start 89.06863 143.8) (end 87.50863 142.24) (width 0.25) (layer B.Cu) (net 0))
 (segment (start 90.2 143.8) (end 89.06863 143.8) (width 0.25) (layer B.Cu) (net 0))
 (segment (start 87.50863 142.24) (end 77.47 142.24) (width 0.25) (layer B.Cu) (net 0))
 (segment (start 74.93 139.7) (end 74.93 138.43) (width 0.25) (layer B.Cu) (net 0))
 (segment (start 77.47 142.24) (end 74.93 139.7) (width 0.25) (layer B.Cu) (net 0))
 (segment (start 76.424594 135.89) (end 80.01 135.89) (width 0.25) (layer F.Cu) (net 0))
 (segment (start 75.884594 136.43) (end 76.424594 135.89) (width 0.25) (layer F.Cu) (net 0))
 (segment (start 74.93 136.43) (end 75.884594 136.43) (width 0.25) (layer F.Cu) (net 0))
 (segment (start 80 122.7) (end 80.01 135.89) (width 0.25) (layer F.Cu) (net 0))
 (segment (start 80.01 135.89) (end 80 139) (width 0.25) (layer F.Cu) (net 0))
 (segment (start 75.4 133.96) (end 74.93 134.43) (width 0.25) (layer F.Cu) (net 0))
 (segment (start 75.4 111.56) (end 75.4 133.96) (width 0.25) (layer F.Cu) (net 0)))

